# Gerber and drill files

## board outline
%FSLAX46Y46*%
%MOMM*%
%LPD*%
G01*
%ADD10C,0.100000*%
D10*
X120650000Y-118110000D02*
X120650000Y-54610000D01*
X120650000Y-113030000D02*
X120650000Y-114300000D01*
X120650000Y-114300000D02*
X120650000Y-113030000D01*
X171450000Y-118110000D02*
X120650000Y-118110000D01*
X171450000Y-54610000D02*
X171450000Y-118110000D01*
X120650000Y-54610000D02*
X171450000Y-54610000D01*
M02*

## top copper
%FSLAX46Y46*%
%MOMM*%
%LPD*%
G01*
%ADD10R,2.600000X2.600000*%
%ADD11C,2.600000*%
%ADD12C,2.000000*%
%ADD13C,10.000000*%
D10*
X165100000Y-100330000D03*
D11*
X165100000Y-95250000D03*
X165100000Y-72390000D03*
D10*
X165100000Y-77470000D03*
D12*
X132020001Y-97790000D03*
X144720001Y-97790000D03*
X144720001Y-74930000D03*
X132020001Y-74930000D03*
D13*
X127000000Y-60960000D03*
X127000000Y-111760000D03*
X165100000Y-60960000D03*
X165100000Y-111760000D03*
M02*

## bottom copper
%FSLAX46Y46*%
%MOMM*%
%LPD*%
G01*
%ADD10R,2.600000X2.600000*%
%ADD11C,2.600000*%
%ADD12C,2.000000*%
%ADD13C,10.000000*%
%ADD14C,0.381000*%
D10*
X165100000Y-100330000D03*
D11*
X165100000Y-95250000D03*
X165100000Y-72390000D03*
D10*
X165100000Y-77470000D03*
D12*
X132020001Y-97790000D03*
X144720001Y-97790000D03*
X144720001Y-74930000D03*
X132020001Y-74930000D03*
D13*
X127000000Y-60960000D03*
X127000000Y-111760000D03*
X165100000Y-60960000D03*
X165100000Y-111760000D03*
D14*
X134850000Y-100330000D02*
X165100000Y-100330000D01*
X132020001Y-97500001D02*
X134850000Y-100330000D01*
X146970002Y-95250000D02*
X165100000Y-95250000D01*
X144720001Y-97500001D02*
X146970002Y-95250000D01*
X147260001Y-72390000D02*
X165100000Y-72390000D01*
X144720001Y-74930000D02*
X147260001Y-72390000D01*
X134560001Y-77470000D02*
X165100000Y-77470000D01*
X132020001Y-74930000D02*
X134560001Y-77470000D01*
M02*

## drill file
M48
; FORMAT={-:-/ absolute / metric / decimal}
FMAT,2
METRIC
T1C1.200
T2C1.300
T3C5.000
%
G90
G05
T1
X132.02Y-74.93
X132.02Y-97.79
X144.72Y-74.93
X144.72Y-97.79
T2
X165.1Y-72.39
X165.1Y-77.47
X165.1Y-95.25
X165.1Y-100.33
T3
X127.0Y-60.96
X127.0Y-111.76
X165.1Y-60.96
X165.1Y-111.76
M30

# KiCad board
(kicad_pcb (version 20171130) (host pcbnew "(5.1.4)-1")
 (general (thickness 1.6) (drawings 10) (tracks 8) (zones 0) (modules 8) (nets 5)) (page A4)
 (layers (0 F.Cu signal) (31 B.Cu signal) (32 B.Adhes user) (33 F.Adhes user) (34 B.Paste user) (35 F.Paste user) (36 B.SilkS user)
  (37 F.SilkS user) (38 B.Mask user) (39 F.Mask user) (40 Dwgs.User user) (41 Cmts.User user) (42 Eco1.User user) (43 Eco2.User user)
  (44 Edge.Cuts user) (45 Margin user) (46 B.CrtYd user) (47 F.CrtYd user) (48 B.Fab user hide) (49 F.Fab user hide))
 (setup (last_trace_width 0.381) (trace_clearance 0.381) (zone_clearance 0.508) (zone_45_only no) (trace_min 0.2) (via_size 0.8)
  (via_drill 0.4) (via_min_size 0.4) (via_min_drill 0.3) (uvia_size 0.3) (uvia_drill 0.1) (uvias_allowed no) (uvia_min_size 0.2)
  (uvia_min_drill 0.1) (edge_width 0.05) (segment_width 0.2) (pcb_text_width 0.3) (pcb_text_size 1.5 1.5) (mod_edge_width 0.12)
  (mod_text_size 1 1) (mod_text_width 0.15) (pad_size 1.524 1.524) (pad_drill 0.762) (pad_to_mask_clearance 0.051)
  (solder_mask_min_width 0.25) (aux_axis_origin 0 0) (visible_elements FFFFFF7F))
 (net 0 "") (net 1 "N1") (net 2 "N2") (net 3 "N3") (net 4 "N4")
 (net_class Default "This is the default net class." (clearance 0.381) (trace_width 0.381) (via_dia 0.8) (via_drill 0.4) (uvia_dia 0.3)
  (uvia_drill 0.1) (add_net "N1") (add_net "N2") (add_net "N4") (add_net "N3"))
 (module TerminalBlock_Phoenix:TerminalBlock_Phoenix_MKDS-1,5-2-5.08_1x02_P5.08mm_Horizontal (layer F.Cu) (at 165.1 100.33 90)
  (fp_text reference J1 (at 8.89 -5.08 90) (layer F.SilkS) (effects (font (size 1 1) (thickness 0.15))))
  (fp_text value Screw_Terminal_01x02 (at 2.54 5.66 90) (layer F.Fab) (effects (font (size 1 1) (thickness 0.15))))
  (pad 1 thru_hole rect (at 0 0 90) (size 2.6 2.6) (drill 1.3) (layers *.Cu *.Mask) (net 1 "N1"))
  (pad 2 thru_hole circle (at 5.08 0 90) (size 2.6 2.6) (drill 1.3) (layers *.Cu *.Mask) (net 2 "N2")))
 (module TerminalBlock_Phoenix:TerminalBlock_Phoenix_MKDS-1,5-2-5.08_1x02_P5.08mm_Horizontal (layer F.Cu) (at 165.1 77.47 90)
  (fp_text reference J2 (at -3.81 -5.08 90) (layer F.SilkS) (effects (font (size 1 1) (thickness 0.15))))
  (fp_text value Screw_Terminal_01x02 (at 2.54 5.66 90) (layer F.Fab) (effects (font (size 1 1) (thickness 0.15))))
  (pad 2 thru_hole circle (at 5.08 0 90) (size 2.6 2.6) (drill 1.3) (layers *.Cu *.Mask) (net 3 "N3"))
  (pad 1 thru_hole rect (at 0 0 90) (size 2.6 2.6) (drill 1.3) (layers *.Cu *.Mask) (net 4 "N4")))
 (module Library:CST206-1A (layer F.Cu) (at 138.370001 97.79)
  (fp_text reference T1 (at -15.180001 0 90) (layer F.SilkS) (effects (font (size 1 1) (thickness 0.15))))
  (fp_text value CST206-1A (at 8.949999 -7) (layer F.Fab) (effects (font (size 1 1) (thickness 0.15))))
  (pad 1 thru_hole circle (at -6.35 0) (size 2 2) (drill 1.2) (layers *.Cu *.Mask) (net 1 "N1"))
  (pad 2 thru_hole circle (at 6.35 0) (size 2 2) (drill 1.2) (layers *.Cu *.Mask) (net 2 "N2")))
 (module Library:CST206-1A (layer F.Cu) (at 138.370001 74.93)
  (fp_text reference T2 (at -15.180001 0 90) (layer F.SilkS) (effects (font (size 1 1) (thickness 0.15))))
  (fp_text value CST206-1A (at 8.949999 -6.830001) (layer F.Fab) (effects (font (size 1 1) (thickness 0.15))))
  (pad 2 thru_hole circle (at 6.35 0) (size 2 2) (drill 1.2) (layers *.Cu *.Mask) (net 3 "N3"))
  (pad 1 thru_hole circle (at -6.35 0) (size 2 2) (drill 1.2) (layers *.Cu *.Mask) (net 4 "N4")))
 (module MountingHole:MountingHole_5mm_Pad (layer F.Cu) (at 127 60.96 90)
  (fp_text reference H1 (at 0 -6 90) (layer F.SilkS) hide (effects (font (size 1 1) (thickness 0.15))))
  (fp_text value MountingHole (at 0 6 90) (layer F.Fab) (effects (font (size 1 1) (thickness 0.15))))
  (pad 1 thru_hole circle (at 0 0 90) (size 10 10) (drill 5) (layers *.Cu *.Mask)))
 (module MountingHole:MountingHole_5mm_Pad (layer F.Cu) (at 127 111.76 90)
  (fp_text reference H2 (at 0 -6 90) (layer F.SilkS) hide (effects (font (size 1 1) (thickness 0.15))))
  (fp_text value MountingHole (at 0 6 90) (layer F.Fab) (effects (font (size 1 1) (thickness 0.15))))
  (pad 1 thru_hole circle (at 0 0 90) (size 10 10) (drill 5) (layers *.Cu *.Mask)))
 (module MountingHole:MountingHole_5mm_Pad (layer F.Cu) (at 165.1 60.96 90)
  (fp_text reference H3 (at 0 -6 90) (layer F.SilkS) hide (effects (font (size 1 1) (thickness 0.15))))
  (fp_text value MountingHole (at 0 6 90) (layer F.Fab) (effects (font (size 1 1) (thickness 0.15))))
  (pad 1 thru_hole circle (at 0 0 90) (size 10 10) (drill 5) (layers *.Cu *.Mask)))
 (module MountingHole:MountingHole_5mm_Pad (layer F.Cu) (at 165.1 111.76 90)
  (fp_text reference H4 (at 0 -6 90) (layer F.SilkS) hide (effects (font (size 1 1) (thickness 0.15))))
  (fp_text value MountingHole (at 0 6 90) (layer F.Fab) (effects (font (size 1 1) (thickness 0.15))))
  (pad 1 thru_hole circle (at 0 0 90) (size 10 10) (drill 5) (layers *.Cu *.Mask)))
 (gr_line (start 120.65 118.11) (end 120.65 54.61) (layer Edge.Cuts) (width 0.1))
 (gr_line (start 120.65 113.03) (end 120.65 114.3) (layer Edge.Cuts) (width 0.1))
 (gr_line (start 120.65 114.3) (end 120.65 113.03) (layer Edge.Cuts) (width 0.1))
 (gr_line (start 171.45 118.11) (end 120.65 118.11) (layer Edge.Cuts) (width 0.1))
 (gr_line (start 171.45 54.61) (end 171.45 118.11) (layer Edge.Cuts) (width 0.1))
 (gr_line (start 120.65 54.61) (end 171.45 54.61) (layer Edge.Cuts) (width 0.1))
 (segment (start 134.85 100.33) (end 165.1 100.33) (width 0.381) (layer B.Cu) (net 1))
 (segment (start 132.020001 97.500001) (end 134.85 100.33) (width 0.381) (layer B.Cu) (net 1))
 (segment (start 146.970002 95.25) (end 165.1 95.25) (width 0.381) (layer B.Cu) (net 2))
 (segment (start 144.720001 97.500001) (end 146.970002 95.25) (width 0.381) (layer B.Cu) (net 2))
 (segment (start 147.260001 72.39) (end 165.1 72.39) (width 0.381) (layer B.Cu) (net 3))
 (segment (start 144.720001 74.93) (end 147.260001 72.39) (width 0.381) (layer B.Cu) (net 3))
 (segment (start 134.560001 77.47) (end 165.1 77.47) (width 0.381) (layer B.Cu) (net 4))
 (segment (start 132.020001 74.93) (end 134.560001 77.47) (width 0.381) (layer B.Cu) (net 4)))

